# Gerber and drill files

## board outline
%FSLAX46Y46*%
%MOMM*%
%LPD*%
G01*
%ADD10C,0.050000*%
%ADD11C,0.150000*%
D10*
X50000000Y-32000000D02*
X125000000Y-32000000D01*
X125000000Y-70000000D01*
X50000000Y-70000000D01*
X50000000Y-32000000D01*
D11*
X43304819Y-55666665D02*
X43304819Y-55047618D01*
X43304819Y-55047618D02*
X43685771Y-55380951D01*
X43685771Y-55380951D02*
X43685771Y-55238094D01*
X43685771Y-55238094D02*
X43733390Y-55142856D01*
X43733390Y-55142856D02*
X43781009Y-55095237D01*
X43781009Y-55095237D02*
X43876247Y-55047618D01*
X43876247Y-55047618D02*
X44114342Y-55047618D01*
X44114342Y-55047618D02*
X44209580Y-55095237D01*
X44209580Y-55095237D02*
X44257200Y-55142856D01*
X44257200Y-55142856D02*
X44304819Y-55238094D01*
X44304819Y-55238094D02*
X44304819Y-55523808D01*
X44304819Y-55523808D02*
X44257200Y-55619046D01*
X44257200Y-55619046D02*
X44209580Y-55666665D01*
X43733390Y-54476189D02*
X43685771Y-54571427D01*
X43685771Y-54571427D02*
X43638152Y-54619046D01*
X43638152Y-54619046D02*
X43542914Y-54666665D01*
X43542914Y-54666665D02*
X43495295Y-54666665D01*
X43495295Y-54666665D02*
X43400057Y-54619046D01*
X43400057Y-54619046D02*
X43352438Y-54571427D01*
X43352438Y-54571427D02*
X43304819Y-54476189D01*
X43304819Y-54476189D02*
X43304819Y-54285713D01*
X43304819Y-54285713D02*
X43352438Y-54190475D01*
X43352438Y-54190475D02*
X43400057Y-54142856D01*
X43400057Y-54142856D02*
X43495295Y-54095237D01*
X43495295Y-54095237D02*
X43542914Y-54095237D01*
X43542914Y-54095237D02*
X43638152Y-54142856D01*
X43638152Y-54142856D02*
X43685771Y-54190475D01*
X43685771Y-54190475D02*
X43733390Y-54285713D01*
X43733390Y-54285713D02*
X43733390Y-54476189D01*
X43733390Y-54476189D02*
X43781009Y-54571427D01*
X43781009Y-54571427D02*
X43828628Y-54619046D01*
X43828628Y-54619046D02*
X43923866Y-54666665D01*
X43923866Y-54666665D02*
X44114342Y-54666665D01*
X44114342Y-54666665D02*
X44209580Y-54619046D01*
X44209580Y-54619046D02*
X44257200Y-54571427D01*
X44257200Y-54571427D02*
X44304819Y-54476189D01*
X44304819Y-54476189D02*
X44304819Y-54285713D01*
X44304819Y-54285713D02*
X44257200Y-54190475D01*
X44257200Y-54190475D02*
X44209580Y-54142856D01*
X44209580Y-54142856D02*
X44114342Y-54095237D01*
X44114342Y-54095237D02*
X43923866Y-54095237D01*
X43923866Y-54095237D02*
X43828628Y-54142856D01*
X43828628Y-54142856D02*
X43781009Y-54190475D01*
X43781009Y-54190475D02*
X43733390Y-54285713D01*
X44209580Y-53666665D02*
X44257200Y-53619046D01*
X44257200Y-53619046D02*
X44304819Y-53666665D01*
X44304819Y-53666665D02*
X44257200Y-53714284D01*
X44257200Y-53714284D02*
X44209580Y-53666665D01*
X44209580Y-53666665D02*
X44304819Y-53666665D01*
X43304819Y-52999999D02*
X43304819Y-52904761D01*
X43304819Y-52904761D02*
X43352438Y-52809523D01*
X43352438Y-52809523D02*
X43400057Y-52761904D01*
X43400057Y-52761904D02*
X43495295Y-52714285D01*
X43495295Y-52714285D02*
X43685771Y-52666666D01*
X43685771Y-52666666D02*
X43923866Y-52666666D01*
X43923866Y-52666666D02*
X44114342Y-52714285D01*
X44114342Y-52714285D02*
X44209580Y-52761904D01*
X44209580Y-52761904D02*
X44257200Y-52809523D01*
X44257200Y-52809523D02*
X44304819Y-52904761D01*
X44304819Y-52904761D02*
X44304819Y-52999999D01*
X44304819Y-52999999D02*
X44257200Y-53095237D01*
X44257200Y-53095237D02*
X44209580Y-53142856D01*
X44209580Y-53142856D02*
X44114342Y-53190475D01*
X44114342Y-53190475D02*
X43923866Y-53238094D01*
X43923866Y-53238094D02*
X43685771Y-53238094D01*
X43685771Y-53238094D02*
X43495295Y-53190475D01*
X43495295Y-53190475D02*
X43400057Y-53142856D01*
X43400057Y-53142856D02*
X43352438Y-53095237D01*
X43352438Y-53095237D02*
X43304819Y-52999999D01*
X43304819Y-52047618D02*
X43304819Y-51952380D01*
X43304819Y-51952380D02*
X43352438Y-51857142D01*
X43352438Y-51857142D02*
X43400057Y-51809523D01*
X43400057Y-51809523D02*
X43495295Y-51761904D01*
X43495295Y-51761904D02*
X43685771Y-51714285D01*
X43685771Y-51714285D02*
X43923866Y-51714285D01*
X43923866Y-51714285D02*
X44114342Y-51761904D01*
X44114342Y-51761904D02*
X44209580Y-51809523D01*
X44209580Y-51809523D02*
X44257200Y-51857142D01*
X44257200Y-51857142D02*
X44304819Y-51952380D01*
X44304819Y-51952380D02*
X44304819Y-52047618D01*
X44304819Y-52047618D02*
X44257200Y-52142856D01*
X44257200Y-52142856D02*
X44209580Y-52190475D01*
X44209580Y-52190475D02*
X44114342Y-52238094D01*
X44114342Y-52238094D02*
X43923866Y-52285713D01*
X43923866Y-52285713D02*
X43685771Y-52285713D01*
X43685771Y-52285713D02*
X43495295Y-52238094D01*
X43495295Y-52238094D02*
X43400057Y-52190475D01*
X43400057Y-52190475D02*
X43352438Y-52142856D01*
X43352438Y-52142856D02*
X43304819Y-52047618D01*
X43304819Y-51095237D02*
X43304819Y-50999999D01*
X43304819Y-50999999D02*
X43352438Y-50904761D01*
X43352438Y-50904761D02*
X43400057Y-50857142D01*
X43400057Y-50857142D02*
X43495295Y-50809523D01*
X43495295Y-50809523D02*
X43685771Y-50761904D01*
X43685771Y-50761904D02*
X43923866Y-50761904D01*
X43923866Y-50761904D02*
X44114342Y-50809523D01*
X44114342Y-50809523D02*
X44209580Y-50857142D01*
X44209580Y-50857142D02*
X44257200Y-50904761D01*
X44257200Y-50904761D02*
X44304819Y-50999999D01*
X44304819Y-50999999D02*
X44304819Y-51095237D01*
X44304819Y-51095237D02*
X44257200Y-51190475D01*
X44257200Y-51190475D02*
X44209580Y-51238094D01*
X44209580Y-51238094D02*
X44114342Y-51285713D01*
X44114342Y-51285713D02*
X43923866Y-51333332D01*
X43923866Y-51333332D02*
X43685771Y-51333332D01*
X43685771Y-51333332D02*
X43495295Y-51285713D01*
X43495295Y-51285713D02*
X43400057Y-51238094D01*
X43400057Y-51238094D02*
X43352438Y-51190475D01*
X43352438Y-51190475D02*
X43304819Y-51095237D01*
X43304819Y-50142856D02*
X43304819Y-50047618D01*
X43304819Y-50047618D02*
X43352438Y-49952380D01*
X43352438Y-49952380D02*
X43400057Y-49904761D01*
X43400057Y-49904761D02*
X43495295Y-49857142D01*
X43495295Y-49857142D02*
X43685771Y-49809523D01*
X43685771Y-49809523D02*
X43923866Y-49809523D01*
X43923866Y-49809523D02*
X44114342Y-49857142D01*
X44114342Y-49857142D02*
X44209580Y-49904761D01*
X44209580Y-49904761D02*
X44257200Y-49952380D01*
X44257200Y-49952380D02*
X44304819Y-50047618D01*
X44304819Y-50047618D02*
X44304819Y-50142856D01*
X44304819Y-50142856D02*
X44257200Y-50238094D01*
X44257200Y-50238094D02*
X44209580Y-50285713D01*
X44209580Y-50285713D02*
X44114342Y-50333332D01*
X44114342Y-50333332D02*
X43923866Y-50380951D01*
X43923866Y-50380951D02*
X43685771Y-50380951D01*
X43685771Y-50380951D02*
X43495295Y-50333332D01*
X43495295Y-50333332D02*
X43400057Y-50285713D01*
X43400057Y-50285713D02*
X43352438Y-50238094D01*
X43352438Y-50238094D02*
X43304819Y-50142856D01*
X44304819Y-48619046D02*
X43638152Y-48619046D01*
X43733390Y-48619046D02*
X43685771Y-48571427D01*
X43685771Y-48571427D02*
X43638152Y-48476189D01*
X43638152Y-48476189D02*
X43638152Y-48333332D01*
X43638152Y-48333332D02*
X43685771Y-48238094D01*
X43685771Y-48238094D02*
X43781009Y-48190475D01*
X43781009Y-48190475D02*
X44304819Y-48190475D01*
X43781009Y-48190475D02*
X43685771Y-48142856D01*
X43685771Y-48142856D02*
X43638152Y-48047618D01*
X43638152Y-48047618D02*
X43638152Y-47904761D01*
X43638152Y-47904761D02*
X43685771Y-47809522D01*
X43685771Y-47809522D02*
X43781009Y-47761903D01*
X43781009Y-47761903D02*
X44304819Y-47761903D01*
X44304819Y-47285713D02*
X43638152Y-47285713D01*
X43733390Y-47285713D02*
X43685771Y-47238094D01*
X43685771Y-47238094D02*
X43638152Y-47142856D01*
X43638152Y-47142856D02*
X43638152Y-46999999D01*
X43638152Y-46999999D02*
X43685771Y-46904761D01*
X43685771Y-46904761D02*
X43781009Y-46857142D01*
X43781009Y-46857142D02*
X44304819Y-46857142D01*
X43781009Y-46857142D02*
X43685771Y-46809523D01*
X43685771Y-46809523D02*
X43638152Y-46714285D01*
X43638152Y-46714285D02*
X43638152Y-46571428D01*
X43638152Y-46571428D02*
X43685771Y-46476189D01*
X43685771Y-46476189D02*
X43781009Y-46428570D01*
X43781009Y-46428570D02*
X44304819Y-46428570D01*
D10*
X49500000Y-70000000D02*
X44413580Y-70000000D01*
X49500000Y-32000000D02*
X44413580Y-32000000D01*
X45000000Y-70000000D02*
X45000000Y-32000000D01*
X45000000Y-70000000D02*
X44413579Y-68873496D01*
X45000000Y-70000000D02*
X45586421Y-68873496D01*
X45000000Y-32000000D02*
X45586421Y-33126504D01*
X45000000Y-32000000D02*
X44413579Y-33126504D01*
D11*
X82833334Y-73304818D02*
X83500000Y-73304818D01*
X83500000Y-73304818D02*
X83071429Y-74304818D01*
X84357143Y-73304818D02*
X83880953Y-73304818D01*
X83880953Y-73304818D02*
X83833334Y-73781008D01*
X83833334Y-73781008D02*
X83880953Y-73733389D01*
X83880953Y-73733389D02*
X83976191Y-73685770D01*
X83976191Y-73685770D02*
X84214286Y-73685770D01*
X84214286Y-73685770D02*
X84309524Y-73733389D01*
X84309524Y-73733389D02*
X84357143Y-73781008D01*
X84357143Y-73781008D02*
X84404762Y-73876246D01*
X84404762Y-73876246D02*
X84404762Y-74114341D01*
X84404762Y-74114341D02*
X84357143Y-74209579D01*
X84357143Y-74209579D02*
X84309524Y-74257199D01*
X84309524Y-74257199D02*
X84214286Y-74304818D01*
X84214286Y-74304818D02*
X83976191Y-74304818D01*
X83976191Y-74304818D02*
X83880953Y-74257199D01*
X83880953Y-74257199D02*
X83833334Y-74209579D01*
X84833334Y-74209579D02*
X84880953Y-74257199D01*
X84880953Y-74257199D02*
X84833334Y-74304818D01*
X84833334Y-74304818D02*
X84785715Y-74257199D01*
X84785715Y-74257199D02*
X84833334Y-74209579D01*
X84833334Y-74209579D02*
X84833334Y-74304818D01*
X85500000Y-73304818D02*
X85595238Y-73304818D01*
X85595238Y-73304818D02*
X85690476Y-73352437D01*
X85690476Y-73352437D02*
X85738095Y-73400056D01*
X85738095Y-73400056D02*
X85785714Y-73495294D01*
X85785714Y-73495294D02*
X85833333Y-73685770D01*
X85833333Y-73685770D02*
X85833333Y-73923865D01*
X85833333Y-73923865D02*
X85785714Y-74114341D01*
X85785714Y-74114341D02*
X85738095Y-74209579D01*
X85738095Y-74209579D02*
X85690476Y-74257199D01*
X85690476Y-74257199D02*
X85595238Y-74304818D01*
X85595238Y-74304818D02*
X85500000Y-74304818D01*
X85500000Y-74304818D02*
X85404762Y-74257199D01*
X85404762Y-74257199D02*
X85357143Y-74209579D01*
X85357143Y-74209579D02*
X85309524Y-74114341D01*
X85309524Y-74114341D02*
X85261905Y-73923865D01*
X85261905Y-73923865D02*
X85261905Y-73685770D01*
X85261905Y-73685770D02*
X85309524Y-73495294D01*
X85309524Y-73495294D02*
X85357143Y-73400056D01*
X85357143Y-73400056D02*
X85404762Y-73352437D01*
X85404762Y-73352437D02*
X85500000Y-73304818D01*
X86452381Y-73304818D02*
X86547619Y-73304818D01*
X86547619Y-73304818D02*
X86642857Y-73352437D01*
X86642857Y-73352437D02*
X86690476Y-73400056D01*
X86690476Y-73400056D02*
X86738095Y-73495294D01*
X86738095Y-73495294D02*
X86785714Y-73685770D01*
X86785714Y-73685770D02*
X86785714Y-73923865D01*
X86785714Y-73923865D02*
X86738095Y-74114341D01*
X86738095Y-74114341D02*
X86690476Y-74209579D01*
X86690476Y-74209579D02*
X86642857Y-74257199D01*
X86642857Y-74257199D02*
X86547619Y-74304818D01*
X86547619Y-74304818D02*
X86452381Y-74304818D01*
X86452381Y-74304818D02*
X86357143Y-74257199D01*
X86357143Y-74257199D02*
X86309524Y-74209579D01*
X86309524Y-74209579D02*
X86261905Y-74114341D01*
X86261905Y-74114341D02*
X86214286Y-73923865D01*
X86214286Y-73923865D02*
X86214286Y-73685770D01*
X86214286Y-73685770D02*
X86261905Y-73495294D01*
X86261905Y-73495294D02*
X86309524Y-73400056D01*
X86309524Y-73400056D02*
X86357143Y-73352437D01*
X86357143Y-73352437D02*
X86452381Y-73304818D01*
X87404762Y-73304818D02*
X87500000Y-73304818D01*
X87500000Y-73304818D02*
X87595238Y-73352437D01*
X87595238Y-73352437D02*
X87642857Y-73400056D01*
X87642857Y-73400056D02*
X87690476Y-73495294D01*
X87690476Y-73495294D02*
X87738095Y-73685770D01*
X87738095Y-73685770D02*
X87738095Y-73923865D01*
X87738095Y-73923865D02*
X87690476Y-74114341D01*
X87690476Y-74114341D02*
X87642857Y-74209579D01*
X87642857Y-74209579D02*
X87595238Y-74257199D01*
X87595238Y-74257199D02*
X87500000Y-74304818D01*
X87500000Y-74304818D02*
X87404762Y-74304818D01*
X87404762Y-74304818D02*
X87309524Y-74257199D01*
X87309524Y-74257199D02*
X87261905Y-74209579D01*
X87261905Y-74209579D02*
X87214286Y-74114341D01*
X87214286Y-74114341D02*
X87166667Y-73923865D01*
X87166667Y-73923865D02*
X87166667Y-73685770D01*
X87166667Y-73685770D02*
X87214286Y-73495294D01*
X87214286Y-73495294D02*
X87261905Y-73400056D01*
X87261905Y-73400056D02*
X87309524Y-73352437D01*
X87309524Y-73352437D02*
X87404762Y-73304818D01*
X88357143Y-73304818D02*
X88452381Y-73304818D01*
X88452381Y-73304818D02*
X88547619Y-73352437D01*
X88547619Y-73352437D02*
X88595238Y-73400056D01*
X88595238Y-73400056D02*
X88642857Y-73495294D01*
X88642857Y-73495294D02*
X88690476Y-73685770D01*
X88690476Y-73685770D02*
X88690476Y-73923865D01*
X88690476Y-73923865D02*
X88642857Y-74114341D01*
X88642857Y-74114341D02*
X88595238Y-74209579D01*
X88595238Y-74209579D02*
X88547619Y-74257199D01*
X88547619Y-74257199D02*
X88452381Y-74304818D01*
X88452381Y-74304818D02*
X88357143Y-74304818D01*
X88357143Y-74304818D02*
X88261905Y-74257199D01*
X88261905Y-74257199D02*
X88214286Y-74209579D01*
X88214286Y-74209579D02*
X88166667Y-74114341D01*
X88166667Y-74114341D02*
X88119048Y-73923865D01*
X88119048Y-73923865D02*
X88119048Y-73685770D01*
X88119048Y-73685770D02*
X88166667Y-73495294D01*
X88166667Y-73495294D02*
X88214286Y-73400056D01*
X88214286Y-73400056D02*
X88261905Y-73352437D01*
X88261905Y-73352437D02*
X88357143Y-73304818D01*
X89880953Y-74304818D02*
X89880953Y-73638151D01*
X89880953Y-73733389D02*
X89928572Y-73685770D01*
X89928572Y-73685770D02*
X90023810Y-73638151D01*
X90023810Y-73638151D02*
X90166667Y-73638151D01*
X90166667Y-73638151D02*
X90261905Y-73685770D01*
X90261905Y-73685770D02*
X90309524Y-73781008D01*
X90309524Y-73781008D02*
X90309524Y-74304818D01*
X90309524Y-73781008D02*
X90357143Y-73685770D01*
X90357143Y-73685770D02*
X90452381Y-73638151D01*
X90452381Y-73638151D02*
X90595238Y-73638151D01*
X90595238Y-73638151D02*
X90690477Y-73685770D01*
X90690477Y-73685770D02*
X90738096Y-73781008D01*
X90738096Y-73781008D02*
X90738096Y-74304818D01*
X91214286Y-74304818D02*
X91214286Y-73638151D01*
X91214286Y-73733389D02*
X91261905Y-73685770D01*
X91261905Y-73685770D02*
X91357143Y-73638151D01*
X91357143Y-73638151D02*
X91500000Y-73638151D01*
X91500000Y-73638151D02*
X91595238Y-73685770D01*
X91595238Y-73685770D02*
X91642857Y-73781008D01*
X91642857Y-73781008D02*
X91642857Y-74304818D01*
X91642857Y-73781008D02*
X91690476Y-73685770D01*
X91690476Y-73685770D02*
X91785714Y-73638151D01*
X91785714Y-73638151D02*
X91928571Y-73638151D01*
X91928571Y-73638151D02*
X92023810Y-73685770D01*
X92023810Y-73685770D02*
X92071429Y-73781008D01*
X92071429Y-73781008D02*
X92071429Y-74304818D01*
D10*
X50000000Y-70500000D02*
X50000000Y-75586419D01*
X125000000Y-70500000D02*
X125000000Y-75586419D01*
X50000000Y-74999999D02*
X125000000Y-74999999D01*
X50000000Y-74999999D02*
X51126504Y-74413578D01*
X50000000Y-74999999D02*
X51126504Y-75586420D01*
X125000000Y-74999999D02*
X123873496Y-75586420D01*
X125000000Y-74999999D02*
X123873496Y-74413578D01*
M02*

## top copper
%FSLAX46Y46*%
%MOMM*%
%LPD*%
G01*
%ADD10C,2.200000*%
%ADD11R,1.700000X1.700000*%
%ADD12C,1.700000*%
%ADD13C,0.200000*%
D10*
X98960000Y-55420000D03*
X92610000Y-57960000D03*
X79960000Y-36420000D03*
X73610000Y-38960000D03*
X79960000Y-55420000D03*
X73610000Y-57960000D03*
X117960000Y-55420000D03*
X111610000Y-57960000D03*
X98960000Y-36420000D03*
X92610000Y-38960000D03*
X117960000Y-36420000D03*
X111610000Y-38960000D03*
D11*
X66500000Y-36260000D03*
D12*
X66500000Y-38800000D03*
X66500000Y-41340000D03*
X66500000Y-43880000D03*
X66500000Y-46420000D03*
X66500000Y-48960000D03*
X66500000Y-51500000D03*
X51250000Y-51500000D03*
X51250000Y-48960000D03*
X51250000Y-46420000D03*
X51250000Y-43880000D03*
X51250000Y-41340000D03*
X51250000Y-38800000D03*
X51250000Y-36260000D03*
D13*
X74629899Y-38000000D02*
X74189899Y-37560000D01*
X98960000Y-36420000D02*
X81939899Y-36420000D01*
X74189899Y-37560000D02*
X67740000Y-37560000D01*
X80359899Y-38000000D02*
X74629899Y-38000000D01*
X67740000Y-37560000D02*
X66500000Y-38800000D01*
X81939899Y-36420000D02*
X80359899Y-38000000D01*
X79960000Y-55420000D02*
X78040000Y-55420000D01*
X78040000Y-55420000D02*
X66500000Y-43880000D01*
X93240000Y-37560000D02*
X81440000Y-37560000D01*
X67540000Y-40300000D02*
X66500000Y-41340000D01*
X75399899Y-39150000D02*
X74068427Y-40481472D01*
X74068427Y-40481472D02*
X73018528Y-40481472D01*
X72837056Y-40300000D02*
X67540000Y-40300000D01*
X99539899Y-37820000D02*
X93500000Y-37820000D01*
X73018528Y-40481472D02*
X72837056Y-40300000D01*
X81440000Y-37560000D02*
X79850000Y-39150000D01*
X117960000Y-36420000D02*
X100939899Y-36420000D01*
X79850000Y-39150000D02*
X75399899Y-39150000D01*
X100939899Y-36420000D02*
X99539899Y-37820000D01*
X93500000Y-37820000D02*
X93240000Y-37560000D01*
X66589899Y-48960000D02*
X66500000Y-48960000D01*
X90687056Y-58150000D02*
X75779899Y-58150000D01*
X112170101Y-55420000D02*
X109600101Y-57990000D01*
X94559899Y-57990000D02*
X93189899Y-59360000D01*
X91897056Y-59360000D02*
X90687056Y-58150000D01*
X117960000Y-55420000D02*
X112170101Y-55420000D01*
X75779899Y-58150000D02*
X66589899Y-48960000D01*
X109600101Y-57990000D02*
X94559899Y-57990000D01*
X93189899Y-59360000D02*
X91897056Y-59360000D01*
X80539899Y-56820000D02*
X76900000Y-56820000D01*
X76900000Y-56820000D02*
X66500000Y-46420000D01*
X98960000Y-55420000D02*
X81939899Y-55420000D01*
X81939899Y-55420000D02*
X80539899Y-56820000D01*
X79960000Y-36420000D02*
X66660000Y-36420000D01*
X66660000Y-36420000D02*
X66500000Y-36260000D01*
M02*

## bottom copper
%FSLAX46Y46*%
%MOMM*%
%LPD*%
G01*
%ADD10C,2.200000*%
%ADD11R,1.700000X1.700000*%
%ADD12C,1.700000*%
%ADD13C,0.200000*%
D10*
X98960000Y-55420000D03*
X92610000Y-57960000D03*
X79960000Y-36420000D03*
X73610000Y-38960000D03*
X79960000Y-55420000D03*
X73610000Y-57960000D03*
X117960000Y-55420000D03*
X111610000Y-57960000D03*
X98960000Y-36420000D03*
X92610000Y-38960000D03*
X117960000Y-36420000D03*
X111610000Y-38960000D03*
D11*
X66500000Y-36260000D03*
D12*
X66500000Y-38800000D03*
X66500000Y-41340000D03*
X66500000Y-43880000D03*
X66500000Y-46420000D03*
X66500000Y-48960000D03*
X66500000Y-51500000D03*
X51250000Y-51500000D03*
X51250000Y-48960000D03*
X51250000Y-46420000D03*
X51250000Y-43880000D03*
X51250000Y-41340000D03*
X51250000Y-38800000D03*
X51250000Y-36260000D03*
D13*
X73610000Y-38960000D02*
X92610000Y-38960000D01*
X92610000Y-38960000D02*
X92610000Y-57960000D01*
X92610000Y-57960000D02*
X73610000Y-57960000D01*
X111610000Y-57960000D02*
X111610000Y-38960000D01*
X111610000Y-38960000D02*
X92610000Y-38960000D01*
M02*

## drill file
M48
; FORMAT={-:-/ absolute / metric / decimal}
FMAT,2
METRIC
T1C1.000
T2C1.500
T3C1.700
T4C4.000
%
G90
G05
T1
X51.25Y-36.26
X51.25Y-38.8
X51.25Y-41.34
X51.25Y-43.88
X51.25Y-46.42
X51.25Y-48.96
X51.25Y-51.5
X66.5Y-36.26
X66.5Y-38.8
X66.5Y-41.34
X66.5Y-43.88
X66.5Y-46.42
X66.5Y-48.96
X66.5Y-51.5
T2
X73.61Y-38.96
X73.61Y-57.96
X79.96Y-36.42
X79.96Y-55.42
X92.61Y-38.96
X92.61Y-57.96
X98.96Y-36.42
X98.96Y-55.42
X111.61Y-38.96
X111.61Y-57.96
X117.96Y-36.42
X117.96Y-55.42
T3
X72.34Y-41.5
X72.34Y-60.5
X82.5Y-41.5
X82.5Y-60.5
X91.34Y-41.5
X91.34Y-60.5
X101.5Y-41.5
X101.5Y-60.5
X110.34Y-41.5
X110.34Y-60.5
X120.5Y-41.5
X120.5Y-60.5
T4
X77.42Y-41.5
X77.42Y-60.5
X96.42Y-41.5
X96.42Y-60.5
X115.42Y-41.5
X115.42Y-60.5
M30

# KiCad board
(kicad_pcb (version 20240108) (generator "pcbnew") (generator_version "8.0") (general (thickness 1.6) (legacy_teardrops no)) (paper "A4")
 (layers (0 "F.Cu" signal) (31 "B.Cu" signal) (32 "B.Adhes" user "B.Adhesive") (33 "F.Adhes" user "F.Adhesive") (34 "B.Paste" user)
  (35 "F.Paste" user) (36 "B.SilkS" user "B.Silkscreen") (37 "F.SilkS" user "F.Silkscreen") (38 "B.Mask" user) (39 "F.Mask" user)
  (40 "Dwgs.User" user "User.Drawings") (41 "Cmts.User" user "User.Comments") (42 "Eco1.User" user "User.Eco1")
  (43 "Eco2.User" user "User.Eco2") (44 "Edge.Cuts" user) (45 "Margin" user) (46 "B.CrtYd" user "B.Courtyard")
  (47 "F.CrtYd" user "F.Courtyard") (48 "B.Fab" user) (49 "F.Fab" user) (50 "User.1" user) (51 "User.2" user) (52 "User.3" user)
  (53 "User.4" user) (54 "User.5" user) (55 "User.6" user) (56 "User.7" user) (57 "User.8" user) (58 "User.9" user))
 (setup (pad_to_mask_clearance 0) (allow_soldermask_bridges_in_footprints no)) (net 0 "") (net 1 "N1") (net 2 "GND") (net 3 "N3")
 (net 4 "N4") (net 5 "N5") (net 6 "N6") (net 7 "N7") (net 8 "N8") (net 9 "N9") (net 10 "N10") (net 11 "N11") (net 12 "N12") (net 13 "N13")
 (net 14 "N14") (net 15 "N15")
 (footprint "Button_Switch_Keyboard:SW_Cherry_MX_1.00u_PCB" (layer "F.Cu") (at 98.96 55.42)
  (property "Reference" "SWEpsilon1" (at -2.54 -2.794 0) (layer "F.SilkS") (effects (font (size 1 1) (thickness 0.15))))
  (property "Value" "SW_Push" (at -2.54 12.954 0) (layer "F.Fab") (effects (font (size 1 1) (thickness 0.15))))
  (pad "" np_thru_hole circle (at -7.62 5.08) (size 1.7 1.7) (drill 1.7) (layers "*.Cu" "*.Mask"))
  (pad "" np_thru_hole circle (at -2.54 5.08) (size 4 4) (drill 4) (layers "*.Cu" "*.Mask"))
  (pad "" np_thru_hole circle (at 2.54 5.08) (size 1.7 1.7) (drill 1.7) (layers "*.Cu" "*.Mask"))
  (pad "1" thru_hole circle (at 0 0) (size 2.2 2.2) (drill 1.5) (layers "*.Cu" "*.Mask") (remove_unused_layers no) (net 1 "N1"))
  (pad "2" thru_hole circle (at -6.35 2.54) (size 2.2 2.2) (drill 1.5) (layers "*.Cu" "*.Mask") (remove_unused_layers no) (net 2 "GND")))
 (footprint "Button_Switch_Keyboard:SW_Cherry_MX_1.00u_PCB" (layer "F.Cu") (at 79.96 36.42)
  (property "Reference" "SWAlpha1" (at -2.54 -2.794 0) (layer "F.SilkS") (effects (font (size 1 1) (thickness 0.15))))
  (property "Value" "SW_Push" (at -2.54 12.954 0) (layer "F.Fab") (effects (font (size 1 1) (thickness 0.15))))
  (pad "" np_thru_hole circle (at -7.62 5.08) (size 1.7 1.7) (drill 1.7) (layers "*.Cu" "*.Mask"))
  (pad "" np_thru_hole circle (at -2.54 5.08) (size 4 4) (drill 4) (layers "*.Cu" "*.Mask"))
  (pad "" np_thru_hole circle (at 2.54 5.08) (size 1.7 1.7) (drill 1.7) (layers "*.Cu" "*.Mask"))
  (pad "1" thru_hole circle (at 0 0) (size 2.2 2.2) (drill 1.5) (layers "*.Cu" "*.Mask") (remove_unused_layers no) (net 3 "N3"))
  (pad "2" thru_hole circle (at -6.35 2.54) (size 2.2 2.2) (drill 1.5) (layers "*.Cu" "*.Mask") (remove_unused_layers no) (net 2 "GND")))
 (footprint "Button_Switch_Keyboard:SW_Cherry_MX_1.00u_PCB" (layer "F.Cu") (at 79.96 55.42)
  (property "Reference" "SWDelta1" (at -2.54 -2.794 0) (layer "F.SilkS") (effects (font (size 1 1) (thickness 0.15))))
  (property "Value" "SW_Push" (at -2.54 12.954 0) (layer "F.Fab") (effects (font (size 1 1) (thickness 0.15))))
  (pad "" np_thru_hole circle (at -7.62 5.08) (size 1.7 1.7) (drill 1.7) (layers "*.Cu" "*.Mask"))
  (pad "" np_thru_hole circle (at -2.54 5.08) (size 4 4) (drill 4) (layers "*.Cu" "*.Mask"))
  (pad "" np_thru_hole circle (at 2.54 5.08) (size 1.7 1.7) (drill 1.7) (layers "*.Cu" "*.Mask"))
  (pad "1" thru_hole circle (at 0 0) (size 2.2 2.2) (drill 1.5) (layers "*.Cu" "*.Mask") (remove_unused_layers no) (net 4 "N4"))
  (pad "2" thru_hole circle (at -6.35 2.54) (size 2.2 2.2) (drill 1.5) (layers "*.Cu" "*.Mask") (remove_unused_layers no) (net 2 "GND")))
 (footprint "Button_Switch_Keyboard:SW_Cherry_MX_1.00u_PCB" (layer "F.Cu") (at 117.96 55.42)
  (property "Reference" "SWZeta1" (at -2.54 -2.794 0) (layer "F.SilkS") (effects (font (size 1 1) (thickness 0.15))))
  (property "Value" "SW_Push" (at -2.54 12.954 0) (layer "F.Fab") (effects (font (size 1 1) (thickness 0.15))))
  (pad "" np_thru_hole circle (at -7.62 5.08) (size 1.7 1.7) (drill 1.7) (layers "*.Cu" "*.Mask"))
  (pad "" np_thru_hole circle (at -2.54 5.08) (size 4 4) (drill 4) (layers "*.Cu" "*.Mask"))
  (pad "" np_thru_hole circle (at 2.54 5.08) (size 1.7 1.7) (drill 1.7) (layers "*.Cu" "*.Mask"))
  (pad "1" thru_hole circle (at 0 0) (size 2.2 2.2) (drill 1.5) (layers "*.Cu" "*.Mask") (remove_unused_layers no) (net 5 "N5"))
  (pad "2" thru_hole circle (at -6.35 2.54) (size 2.2 2.2) (drill 1.5) (layers "*.Cu" "*.Mask") (remove_unused_layers no) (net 2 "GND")))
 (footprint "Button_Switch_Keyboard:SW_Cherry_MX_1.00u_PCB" (layer "F.Cu") (at 98.96 36.42)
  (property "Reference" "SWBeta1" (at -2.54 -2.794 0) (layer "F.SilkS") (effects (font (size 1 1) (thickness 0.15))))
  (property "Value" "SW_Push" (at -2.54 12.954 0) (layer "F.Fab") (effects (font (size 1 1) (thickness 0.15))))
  (pad "" np_thru_hole circle (at -7.62 5.08) (size 1.7 1.7) (drill 1.7) (layers "*.Cu" "*.Mask"))
  (pad "" np_thru_hole circle (at -2.54 5.08) (size 4 4) (drill 4) (layers "*.Cu" "*.Mask"))
  (pad "" np_thru_hole circle (at 2.54 5.08) (size 1.7 1.7) (drill 1.7) (layers "*.Cu" "*.Mask"))
  (pad "1" thru_hole circle (at 0 0) (size 2.2 2.2) (drill 1.5) (layers "*.Cu" "*.Mask") (remove_unused_layers no) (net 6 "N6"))
  (pad "2" thru_hole circle (at -6.35 2.54) (size 2.2 2.2) (drill 1.5) (layers "*.Cu" "*.Mask") (remove_unused_layers no) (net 2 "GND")))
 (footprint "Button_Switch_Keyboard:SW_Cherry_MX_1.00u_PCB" (layer "F.Cu") (at 117.96 36.42)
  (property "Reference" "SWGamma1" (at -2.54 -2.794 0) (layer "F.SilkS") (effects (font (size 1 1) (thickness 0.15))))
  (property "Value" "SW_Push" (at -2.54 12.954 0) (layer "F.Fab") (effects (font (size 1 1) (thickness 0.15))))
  (pad "" np_thru_hole circle (at -7.62 5.08) (size 1.7 1.7) (drill 1.7) (layers "*.Cu" "*.Mask"))
  (pad "" np_thru_hole circle (at -2.54 5.08) (size 4 4) (drill 4) (layers "*.Cu" "*.Mask"))
  (pad "" np_thru_hole circle (at 2.54 5.08) (size 1.7 1.7) (drill 1.7) (layers "*.Cu" "*.Mask"))
  (pad "1" thru_hole circle (at 0 0) (size 2.2 2.2) (drill 1.5) (layers "*.Cu" "*.Mask") (remove_unused_layers no) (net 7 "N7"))
  (pad "2" thru_hole circle (at -6.35 2.54) (size 2.2 2.2) (drill 1.5) (layers "*.Cu" "*.Mask") (remove_unused_layers no) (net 2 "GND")))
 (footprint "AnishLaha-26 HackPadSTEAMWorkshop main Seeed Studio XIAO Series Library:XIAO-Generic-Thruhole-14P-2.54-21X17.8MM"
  (layer "B.Cu") (at 58.875 43.88 180)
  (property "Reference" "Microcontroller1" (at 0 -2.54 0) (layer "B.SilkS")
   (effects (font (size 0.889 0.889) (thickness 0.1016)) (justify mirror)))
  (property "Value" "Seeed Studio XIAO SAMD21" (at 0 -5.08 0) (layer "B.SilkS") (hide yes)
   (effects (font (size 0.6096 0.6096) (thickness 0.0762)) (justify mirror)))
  (pad "1" thru_hole rect (at -7.625 7.62 180) (size 1.7 1.7) (drill 1) (layers "*.Cu" "*.Mask") (remove_unused_layers no) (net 3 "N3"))
  (pad "2" thru_hole circle (at -7.625 5.08 180) (size 1.7 1.7) (drill 1) (layers "*.Cu" "*.Mask") (remove_unused_layers no) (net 6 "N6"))
  (pad "3" thru_hole circle (at -7.625 2.54 180) (size 1.7 1.7) (drill 1) (layers "*.Cu" "*.Mask") (remove_unused_layers no) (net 7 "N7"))
  (pad "4" thru_hole circle (at -7.625 0 180) (size 1.7 1.7) (drill 1) (layers "*.Cu" "*.Mask") (remove_unused_layers no) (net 4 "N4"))
  (pad "5" thru_hole circle (at -7.625 -2.54 180) (size 1.7 1.7) (drill 1) (layers "*.Cu" "*.Mask") (remove_unused_layers no) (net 1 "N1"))
  (pad "6" thru_hole circle (at -7.625 -5.08) (size 1.7 1.7) (drill 1) (layers "*.Cu" "*.Mask") (remove_unused_layers no) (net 5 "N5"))
  (pad "7" thru_hole circle (at -7.625 -7.62 180) (size 1.7 1.7) (drill 1) (layers "*.Cu" "*.Mask") (remove_unused_layers no) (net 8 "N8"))
  (pad "8" thru_hole circle (at 7.625 -7.62 180) (size 1.7 1.7) (drill 1) (layers "*.Cu" "*.Mask") (remove_unused_layers no) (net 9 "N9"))
  (pad "9" thru_hole circle (at 7.625 -5.08 180) (size 1.7 1.7) (drill 1) (layers "*.Cu" "*.Mask") (remove_unused_layers no) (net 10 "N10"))
  (pad "10" thru_hole circle (at 7.625 -2.54 180) (size 1.7 1.7) (drill 1) (layers "*.Cu" "*.Mask") (remove_unused_layers no) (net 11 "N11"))
  (pad "11" thru_hole circle (at 7.625 0 180) (size 1.7 1.7) (drill 1) (layers "*.Cu" "*.Mask") (remove_unused_layers no) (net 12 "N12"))
  (pad "12" thru_hole circle (at 7.625 2.54 180) (size 1.7 1.7) (drill 1) (layers "*.Cu" "*.Mask") (remove_unused_layers no) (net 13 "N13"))
  (pad "13" thru_hole circle (at 7.625 5.08 180) (size 1.7 1.7) (drill 1) (layers "*.Cu" "*.Mask") (remove_unused_layers no) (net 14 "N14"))
  (pad "14" thru_hole circle (at 7.625 7.62 180) (size 1.7 1.7) (drill 1) (layers "*.Cu" "*.Mask") (remove_unused_layers no) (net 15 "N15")))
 (gr_rect (start 50 32) (end 125 70) (stroke (width 0.05) (type default)) (fill none) (layer "Edge.Cuts"))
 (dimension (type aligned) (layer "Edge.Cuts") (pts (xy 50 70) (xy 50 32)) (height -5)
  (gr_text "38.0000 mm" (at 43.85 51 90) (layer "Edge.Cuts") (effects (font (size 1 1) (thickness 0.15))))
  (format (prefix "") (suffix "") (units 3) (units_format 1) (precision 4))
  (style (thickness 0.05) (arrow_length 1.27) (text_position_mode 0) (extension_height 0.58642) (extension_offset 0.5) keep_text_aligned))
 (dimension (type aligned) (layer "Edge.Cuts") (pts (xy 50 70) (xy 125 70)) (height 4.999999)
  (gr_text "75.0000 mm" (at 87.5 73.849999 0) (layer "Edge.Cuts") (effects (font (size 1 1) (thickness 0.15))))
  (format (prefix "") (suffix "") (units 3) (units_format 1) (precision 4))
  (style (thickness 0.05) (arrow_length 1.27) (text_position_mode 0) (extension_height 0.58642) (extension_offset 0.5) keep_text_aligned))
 (segment (start 73.61 38.96) (end 92.61 38.96) (width 0.2) (layer "B.Cu") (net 2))
 (segment (start 92.61 38.96) (end 92.61 57.96) (width 0.2) (layer "B.Cu") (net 2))
 (segment (start 92.61 57.96) (end 73.61 57.96) (width 0.2) (layer "B.Cu") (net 2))
 (segment (start 111.61 57.96) (end 111.61 38.96) (width 0.2) (layer "B.Cu") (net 2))
 (segment (start 111.61 38.96) (end 92.61 38.96) (width 0.2) (layer "B.Cu") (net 2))
 (segment (start 74.629899 38) (end 74.189899 37.56) (width 0.2) (layer "F.Cu") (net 6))
 (segment (start 98.96 36.42) (end 81.939899 36.42) (width 0.2) (layer "F.Cu") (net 6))
 (segment (start 74.189899 37.56) (end 67.74 37.56) (width 0.2) (layer "F.Cu") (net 6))
 (segment (start 80.359899 38) (end 74.629899 38) (width 0.2) (layer "F.Cu") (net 6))
 (segment (start 67.74 37.56) (end 66.5 38.8) (width 0.2) (layer "F.Cu") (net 6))
 (segment (start 81.939899 36.42) (end 80.359899 38) (width 0.2) (layer "F.Cu") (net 6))
 (segment (start 79.96 55.42) (end 78.04 55.42) (width 0.2) (layer "F.Cu") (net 4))
 (segment (start 78.04 55.42) (end 66.5 43.88) (width 0.2) (layer "F.Cu") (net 4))
 (segment (start 93.24 37.56) (end 81.44 37.56) (width 0.2) (layer "F.Cu") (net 7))
 (segment (start 67.54 40.3) (end 66.5 41.34) (width 0.2) (layer "F.Cu") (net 7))
 (segment (start 75.399899 39.15) (end 74.068427 40.481472) (width 0.2) (layer "F.Cu") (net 7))
 (segment (start 74.068427 40.481472) (end 73.018528 40.481472) (width 0.2) (layer "F.Cu") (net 7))
 (segment (start 72.837056 40.3) (end 67.54 40.3) (width 0.2) (layer "F.Cu") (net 7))
 (segment (start 99.539899 37.82) (end 93.5 37.82) (width 0.2) (layer "F.Cu") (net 7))
 (segment (start 73.018528 40.481472) (end 72.837056 40.3) (width 0.2) (layer "F.Cu") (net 7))
 (segment (start 81.44 37.56) (end 79.85 39.15) (width 0.2) (layer "F.Cu") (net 7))
 (segment (start 117.96 36.42) (end 100.939899 36.42) (width 0.2) (layer "F.Cu") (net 7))
 (segment (start 79.85 39.15) (end 75.399899 39.15) (width 0.2) (layer "F.Cu") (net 7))
 (segment (start 100.939899 36.42) (end 99.539899 37.82) (width 0.2) (layer "F.Cu") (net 7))
 (segment (start 93.5 37.82) (end 93.24 37.56) (width 0.2) (layer "F.Cu") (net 7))
 (segment (start 66.589899 48.96) (end 66.5 48.96) (width 0.2) (layer "F.Cu") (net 5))
 (segment (start 90.687056 58.15) (end 75.779899 58.15) (width 0.2) (layer "F.Cu") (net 5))
 (segment (start 112.170101 55.42) (end 109.600101 57.99) (width 0.2) (layer "F.Cu") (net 5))
 (segment (start 94.559899 57.99) (end 93.189899 59.36) (width 0.2) (layer "F.Cu") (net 5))
 (segment (start 91.897056 59.36) (end 90.687056 58.15) (width 0.2) (layer "F.Cu") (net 5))
 (segment (start 117.96 55.42) (end 112.170101 55.42) (width 0.2) (layer "F.Cu") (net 5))
 (segment (start 75.779899 58.15) (end 66.589899 48.96) (width 0.2) (layer "F.Cu") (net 5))
 (segment (start 109.600101 57.99) (end 94.559899 57.99) (width 0.2) (layer "F.Cu") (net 5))
 (segment (start 93.189899 59.36) (end 91.897056 59.36) (width 0.2) (layer "F.Cu") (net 5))
 (segment (start 80.539899 56.82) (end 76.9 56.82) (width 0.2) (layer "F.Cu") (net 1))
 (segment (start 76.9 56.82) (end 66.5 46.42) (width 0.2) (layer "F.Cu") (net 1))
 (segment (start 98.96 55.42) (end 81.939899 55.42) (width 0.2) (layer "F.Cu") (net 1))
 (segment (start 81.939899 55.42) (end 80.539899 56.82) (width 0.2) (layer "F.Cu") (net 1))
 (segment (start 79.96 36.42) (end 66.66 36.42) (width 0.2) (layer "F.Cu") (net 3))
 (segment (start 66.66 36.42) (end 66.5 36.26) (width 0.2) (layer "F.Cu") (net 3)))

